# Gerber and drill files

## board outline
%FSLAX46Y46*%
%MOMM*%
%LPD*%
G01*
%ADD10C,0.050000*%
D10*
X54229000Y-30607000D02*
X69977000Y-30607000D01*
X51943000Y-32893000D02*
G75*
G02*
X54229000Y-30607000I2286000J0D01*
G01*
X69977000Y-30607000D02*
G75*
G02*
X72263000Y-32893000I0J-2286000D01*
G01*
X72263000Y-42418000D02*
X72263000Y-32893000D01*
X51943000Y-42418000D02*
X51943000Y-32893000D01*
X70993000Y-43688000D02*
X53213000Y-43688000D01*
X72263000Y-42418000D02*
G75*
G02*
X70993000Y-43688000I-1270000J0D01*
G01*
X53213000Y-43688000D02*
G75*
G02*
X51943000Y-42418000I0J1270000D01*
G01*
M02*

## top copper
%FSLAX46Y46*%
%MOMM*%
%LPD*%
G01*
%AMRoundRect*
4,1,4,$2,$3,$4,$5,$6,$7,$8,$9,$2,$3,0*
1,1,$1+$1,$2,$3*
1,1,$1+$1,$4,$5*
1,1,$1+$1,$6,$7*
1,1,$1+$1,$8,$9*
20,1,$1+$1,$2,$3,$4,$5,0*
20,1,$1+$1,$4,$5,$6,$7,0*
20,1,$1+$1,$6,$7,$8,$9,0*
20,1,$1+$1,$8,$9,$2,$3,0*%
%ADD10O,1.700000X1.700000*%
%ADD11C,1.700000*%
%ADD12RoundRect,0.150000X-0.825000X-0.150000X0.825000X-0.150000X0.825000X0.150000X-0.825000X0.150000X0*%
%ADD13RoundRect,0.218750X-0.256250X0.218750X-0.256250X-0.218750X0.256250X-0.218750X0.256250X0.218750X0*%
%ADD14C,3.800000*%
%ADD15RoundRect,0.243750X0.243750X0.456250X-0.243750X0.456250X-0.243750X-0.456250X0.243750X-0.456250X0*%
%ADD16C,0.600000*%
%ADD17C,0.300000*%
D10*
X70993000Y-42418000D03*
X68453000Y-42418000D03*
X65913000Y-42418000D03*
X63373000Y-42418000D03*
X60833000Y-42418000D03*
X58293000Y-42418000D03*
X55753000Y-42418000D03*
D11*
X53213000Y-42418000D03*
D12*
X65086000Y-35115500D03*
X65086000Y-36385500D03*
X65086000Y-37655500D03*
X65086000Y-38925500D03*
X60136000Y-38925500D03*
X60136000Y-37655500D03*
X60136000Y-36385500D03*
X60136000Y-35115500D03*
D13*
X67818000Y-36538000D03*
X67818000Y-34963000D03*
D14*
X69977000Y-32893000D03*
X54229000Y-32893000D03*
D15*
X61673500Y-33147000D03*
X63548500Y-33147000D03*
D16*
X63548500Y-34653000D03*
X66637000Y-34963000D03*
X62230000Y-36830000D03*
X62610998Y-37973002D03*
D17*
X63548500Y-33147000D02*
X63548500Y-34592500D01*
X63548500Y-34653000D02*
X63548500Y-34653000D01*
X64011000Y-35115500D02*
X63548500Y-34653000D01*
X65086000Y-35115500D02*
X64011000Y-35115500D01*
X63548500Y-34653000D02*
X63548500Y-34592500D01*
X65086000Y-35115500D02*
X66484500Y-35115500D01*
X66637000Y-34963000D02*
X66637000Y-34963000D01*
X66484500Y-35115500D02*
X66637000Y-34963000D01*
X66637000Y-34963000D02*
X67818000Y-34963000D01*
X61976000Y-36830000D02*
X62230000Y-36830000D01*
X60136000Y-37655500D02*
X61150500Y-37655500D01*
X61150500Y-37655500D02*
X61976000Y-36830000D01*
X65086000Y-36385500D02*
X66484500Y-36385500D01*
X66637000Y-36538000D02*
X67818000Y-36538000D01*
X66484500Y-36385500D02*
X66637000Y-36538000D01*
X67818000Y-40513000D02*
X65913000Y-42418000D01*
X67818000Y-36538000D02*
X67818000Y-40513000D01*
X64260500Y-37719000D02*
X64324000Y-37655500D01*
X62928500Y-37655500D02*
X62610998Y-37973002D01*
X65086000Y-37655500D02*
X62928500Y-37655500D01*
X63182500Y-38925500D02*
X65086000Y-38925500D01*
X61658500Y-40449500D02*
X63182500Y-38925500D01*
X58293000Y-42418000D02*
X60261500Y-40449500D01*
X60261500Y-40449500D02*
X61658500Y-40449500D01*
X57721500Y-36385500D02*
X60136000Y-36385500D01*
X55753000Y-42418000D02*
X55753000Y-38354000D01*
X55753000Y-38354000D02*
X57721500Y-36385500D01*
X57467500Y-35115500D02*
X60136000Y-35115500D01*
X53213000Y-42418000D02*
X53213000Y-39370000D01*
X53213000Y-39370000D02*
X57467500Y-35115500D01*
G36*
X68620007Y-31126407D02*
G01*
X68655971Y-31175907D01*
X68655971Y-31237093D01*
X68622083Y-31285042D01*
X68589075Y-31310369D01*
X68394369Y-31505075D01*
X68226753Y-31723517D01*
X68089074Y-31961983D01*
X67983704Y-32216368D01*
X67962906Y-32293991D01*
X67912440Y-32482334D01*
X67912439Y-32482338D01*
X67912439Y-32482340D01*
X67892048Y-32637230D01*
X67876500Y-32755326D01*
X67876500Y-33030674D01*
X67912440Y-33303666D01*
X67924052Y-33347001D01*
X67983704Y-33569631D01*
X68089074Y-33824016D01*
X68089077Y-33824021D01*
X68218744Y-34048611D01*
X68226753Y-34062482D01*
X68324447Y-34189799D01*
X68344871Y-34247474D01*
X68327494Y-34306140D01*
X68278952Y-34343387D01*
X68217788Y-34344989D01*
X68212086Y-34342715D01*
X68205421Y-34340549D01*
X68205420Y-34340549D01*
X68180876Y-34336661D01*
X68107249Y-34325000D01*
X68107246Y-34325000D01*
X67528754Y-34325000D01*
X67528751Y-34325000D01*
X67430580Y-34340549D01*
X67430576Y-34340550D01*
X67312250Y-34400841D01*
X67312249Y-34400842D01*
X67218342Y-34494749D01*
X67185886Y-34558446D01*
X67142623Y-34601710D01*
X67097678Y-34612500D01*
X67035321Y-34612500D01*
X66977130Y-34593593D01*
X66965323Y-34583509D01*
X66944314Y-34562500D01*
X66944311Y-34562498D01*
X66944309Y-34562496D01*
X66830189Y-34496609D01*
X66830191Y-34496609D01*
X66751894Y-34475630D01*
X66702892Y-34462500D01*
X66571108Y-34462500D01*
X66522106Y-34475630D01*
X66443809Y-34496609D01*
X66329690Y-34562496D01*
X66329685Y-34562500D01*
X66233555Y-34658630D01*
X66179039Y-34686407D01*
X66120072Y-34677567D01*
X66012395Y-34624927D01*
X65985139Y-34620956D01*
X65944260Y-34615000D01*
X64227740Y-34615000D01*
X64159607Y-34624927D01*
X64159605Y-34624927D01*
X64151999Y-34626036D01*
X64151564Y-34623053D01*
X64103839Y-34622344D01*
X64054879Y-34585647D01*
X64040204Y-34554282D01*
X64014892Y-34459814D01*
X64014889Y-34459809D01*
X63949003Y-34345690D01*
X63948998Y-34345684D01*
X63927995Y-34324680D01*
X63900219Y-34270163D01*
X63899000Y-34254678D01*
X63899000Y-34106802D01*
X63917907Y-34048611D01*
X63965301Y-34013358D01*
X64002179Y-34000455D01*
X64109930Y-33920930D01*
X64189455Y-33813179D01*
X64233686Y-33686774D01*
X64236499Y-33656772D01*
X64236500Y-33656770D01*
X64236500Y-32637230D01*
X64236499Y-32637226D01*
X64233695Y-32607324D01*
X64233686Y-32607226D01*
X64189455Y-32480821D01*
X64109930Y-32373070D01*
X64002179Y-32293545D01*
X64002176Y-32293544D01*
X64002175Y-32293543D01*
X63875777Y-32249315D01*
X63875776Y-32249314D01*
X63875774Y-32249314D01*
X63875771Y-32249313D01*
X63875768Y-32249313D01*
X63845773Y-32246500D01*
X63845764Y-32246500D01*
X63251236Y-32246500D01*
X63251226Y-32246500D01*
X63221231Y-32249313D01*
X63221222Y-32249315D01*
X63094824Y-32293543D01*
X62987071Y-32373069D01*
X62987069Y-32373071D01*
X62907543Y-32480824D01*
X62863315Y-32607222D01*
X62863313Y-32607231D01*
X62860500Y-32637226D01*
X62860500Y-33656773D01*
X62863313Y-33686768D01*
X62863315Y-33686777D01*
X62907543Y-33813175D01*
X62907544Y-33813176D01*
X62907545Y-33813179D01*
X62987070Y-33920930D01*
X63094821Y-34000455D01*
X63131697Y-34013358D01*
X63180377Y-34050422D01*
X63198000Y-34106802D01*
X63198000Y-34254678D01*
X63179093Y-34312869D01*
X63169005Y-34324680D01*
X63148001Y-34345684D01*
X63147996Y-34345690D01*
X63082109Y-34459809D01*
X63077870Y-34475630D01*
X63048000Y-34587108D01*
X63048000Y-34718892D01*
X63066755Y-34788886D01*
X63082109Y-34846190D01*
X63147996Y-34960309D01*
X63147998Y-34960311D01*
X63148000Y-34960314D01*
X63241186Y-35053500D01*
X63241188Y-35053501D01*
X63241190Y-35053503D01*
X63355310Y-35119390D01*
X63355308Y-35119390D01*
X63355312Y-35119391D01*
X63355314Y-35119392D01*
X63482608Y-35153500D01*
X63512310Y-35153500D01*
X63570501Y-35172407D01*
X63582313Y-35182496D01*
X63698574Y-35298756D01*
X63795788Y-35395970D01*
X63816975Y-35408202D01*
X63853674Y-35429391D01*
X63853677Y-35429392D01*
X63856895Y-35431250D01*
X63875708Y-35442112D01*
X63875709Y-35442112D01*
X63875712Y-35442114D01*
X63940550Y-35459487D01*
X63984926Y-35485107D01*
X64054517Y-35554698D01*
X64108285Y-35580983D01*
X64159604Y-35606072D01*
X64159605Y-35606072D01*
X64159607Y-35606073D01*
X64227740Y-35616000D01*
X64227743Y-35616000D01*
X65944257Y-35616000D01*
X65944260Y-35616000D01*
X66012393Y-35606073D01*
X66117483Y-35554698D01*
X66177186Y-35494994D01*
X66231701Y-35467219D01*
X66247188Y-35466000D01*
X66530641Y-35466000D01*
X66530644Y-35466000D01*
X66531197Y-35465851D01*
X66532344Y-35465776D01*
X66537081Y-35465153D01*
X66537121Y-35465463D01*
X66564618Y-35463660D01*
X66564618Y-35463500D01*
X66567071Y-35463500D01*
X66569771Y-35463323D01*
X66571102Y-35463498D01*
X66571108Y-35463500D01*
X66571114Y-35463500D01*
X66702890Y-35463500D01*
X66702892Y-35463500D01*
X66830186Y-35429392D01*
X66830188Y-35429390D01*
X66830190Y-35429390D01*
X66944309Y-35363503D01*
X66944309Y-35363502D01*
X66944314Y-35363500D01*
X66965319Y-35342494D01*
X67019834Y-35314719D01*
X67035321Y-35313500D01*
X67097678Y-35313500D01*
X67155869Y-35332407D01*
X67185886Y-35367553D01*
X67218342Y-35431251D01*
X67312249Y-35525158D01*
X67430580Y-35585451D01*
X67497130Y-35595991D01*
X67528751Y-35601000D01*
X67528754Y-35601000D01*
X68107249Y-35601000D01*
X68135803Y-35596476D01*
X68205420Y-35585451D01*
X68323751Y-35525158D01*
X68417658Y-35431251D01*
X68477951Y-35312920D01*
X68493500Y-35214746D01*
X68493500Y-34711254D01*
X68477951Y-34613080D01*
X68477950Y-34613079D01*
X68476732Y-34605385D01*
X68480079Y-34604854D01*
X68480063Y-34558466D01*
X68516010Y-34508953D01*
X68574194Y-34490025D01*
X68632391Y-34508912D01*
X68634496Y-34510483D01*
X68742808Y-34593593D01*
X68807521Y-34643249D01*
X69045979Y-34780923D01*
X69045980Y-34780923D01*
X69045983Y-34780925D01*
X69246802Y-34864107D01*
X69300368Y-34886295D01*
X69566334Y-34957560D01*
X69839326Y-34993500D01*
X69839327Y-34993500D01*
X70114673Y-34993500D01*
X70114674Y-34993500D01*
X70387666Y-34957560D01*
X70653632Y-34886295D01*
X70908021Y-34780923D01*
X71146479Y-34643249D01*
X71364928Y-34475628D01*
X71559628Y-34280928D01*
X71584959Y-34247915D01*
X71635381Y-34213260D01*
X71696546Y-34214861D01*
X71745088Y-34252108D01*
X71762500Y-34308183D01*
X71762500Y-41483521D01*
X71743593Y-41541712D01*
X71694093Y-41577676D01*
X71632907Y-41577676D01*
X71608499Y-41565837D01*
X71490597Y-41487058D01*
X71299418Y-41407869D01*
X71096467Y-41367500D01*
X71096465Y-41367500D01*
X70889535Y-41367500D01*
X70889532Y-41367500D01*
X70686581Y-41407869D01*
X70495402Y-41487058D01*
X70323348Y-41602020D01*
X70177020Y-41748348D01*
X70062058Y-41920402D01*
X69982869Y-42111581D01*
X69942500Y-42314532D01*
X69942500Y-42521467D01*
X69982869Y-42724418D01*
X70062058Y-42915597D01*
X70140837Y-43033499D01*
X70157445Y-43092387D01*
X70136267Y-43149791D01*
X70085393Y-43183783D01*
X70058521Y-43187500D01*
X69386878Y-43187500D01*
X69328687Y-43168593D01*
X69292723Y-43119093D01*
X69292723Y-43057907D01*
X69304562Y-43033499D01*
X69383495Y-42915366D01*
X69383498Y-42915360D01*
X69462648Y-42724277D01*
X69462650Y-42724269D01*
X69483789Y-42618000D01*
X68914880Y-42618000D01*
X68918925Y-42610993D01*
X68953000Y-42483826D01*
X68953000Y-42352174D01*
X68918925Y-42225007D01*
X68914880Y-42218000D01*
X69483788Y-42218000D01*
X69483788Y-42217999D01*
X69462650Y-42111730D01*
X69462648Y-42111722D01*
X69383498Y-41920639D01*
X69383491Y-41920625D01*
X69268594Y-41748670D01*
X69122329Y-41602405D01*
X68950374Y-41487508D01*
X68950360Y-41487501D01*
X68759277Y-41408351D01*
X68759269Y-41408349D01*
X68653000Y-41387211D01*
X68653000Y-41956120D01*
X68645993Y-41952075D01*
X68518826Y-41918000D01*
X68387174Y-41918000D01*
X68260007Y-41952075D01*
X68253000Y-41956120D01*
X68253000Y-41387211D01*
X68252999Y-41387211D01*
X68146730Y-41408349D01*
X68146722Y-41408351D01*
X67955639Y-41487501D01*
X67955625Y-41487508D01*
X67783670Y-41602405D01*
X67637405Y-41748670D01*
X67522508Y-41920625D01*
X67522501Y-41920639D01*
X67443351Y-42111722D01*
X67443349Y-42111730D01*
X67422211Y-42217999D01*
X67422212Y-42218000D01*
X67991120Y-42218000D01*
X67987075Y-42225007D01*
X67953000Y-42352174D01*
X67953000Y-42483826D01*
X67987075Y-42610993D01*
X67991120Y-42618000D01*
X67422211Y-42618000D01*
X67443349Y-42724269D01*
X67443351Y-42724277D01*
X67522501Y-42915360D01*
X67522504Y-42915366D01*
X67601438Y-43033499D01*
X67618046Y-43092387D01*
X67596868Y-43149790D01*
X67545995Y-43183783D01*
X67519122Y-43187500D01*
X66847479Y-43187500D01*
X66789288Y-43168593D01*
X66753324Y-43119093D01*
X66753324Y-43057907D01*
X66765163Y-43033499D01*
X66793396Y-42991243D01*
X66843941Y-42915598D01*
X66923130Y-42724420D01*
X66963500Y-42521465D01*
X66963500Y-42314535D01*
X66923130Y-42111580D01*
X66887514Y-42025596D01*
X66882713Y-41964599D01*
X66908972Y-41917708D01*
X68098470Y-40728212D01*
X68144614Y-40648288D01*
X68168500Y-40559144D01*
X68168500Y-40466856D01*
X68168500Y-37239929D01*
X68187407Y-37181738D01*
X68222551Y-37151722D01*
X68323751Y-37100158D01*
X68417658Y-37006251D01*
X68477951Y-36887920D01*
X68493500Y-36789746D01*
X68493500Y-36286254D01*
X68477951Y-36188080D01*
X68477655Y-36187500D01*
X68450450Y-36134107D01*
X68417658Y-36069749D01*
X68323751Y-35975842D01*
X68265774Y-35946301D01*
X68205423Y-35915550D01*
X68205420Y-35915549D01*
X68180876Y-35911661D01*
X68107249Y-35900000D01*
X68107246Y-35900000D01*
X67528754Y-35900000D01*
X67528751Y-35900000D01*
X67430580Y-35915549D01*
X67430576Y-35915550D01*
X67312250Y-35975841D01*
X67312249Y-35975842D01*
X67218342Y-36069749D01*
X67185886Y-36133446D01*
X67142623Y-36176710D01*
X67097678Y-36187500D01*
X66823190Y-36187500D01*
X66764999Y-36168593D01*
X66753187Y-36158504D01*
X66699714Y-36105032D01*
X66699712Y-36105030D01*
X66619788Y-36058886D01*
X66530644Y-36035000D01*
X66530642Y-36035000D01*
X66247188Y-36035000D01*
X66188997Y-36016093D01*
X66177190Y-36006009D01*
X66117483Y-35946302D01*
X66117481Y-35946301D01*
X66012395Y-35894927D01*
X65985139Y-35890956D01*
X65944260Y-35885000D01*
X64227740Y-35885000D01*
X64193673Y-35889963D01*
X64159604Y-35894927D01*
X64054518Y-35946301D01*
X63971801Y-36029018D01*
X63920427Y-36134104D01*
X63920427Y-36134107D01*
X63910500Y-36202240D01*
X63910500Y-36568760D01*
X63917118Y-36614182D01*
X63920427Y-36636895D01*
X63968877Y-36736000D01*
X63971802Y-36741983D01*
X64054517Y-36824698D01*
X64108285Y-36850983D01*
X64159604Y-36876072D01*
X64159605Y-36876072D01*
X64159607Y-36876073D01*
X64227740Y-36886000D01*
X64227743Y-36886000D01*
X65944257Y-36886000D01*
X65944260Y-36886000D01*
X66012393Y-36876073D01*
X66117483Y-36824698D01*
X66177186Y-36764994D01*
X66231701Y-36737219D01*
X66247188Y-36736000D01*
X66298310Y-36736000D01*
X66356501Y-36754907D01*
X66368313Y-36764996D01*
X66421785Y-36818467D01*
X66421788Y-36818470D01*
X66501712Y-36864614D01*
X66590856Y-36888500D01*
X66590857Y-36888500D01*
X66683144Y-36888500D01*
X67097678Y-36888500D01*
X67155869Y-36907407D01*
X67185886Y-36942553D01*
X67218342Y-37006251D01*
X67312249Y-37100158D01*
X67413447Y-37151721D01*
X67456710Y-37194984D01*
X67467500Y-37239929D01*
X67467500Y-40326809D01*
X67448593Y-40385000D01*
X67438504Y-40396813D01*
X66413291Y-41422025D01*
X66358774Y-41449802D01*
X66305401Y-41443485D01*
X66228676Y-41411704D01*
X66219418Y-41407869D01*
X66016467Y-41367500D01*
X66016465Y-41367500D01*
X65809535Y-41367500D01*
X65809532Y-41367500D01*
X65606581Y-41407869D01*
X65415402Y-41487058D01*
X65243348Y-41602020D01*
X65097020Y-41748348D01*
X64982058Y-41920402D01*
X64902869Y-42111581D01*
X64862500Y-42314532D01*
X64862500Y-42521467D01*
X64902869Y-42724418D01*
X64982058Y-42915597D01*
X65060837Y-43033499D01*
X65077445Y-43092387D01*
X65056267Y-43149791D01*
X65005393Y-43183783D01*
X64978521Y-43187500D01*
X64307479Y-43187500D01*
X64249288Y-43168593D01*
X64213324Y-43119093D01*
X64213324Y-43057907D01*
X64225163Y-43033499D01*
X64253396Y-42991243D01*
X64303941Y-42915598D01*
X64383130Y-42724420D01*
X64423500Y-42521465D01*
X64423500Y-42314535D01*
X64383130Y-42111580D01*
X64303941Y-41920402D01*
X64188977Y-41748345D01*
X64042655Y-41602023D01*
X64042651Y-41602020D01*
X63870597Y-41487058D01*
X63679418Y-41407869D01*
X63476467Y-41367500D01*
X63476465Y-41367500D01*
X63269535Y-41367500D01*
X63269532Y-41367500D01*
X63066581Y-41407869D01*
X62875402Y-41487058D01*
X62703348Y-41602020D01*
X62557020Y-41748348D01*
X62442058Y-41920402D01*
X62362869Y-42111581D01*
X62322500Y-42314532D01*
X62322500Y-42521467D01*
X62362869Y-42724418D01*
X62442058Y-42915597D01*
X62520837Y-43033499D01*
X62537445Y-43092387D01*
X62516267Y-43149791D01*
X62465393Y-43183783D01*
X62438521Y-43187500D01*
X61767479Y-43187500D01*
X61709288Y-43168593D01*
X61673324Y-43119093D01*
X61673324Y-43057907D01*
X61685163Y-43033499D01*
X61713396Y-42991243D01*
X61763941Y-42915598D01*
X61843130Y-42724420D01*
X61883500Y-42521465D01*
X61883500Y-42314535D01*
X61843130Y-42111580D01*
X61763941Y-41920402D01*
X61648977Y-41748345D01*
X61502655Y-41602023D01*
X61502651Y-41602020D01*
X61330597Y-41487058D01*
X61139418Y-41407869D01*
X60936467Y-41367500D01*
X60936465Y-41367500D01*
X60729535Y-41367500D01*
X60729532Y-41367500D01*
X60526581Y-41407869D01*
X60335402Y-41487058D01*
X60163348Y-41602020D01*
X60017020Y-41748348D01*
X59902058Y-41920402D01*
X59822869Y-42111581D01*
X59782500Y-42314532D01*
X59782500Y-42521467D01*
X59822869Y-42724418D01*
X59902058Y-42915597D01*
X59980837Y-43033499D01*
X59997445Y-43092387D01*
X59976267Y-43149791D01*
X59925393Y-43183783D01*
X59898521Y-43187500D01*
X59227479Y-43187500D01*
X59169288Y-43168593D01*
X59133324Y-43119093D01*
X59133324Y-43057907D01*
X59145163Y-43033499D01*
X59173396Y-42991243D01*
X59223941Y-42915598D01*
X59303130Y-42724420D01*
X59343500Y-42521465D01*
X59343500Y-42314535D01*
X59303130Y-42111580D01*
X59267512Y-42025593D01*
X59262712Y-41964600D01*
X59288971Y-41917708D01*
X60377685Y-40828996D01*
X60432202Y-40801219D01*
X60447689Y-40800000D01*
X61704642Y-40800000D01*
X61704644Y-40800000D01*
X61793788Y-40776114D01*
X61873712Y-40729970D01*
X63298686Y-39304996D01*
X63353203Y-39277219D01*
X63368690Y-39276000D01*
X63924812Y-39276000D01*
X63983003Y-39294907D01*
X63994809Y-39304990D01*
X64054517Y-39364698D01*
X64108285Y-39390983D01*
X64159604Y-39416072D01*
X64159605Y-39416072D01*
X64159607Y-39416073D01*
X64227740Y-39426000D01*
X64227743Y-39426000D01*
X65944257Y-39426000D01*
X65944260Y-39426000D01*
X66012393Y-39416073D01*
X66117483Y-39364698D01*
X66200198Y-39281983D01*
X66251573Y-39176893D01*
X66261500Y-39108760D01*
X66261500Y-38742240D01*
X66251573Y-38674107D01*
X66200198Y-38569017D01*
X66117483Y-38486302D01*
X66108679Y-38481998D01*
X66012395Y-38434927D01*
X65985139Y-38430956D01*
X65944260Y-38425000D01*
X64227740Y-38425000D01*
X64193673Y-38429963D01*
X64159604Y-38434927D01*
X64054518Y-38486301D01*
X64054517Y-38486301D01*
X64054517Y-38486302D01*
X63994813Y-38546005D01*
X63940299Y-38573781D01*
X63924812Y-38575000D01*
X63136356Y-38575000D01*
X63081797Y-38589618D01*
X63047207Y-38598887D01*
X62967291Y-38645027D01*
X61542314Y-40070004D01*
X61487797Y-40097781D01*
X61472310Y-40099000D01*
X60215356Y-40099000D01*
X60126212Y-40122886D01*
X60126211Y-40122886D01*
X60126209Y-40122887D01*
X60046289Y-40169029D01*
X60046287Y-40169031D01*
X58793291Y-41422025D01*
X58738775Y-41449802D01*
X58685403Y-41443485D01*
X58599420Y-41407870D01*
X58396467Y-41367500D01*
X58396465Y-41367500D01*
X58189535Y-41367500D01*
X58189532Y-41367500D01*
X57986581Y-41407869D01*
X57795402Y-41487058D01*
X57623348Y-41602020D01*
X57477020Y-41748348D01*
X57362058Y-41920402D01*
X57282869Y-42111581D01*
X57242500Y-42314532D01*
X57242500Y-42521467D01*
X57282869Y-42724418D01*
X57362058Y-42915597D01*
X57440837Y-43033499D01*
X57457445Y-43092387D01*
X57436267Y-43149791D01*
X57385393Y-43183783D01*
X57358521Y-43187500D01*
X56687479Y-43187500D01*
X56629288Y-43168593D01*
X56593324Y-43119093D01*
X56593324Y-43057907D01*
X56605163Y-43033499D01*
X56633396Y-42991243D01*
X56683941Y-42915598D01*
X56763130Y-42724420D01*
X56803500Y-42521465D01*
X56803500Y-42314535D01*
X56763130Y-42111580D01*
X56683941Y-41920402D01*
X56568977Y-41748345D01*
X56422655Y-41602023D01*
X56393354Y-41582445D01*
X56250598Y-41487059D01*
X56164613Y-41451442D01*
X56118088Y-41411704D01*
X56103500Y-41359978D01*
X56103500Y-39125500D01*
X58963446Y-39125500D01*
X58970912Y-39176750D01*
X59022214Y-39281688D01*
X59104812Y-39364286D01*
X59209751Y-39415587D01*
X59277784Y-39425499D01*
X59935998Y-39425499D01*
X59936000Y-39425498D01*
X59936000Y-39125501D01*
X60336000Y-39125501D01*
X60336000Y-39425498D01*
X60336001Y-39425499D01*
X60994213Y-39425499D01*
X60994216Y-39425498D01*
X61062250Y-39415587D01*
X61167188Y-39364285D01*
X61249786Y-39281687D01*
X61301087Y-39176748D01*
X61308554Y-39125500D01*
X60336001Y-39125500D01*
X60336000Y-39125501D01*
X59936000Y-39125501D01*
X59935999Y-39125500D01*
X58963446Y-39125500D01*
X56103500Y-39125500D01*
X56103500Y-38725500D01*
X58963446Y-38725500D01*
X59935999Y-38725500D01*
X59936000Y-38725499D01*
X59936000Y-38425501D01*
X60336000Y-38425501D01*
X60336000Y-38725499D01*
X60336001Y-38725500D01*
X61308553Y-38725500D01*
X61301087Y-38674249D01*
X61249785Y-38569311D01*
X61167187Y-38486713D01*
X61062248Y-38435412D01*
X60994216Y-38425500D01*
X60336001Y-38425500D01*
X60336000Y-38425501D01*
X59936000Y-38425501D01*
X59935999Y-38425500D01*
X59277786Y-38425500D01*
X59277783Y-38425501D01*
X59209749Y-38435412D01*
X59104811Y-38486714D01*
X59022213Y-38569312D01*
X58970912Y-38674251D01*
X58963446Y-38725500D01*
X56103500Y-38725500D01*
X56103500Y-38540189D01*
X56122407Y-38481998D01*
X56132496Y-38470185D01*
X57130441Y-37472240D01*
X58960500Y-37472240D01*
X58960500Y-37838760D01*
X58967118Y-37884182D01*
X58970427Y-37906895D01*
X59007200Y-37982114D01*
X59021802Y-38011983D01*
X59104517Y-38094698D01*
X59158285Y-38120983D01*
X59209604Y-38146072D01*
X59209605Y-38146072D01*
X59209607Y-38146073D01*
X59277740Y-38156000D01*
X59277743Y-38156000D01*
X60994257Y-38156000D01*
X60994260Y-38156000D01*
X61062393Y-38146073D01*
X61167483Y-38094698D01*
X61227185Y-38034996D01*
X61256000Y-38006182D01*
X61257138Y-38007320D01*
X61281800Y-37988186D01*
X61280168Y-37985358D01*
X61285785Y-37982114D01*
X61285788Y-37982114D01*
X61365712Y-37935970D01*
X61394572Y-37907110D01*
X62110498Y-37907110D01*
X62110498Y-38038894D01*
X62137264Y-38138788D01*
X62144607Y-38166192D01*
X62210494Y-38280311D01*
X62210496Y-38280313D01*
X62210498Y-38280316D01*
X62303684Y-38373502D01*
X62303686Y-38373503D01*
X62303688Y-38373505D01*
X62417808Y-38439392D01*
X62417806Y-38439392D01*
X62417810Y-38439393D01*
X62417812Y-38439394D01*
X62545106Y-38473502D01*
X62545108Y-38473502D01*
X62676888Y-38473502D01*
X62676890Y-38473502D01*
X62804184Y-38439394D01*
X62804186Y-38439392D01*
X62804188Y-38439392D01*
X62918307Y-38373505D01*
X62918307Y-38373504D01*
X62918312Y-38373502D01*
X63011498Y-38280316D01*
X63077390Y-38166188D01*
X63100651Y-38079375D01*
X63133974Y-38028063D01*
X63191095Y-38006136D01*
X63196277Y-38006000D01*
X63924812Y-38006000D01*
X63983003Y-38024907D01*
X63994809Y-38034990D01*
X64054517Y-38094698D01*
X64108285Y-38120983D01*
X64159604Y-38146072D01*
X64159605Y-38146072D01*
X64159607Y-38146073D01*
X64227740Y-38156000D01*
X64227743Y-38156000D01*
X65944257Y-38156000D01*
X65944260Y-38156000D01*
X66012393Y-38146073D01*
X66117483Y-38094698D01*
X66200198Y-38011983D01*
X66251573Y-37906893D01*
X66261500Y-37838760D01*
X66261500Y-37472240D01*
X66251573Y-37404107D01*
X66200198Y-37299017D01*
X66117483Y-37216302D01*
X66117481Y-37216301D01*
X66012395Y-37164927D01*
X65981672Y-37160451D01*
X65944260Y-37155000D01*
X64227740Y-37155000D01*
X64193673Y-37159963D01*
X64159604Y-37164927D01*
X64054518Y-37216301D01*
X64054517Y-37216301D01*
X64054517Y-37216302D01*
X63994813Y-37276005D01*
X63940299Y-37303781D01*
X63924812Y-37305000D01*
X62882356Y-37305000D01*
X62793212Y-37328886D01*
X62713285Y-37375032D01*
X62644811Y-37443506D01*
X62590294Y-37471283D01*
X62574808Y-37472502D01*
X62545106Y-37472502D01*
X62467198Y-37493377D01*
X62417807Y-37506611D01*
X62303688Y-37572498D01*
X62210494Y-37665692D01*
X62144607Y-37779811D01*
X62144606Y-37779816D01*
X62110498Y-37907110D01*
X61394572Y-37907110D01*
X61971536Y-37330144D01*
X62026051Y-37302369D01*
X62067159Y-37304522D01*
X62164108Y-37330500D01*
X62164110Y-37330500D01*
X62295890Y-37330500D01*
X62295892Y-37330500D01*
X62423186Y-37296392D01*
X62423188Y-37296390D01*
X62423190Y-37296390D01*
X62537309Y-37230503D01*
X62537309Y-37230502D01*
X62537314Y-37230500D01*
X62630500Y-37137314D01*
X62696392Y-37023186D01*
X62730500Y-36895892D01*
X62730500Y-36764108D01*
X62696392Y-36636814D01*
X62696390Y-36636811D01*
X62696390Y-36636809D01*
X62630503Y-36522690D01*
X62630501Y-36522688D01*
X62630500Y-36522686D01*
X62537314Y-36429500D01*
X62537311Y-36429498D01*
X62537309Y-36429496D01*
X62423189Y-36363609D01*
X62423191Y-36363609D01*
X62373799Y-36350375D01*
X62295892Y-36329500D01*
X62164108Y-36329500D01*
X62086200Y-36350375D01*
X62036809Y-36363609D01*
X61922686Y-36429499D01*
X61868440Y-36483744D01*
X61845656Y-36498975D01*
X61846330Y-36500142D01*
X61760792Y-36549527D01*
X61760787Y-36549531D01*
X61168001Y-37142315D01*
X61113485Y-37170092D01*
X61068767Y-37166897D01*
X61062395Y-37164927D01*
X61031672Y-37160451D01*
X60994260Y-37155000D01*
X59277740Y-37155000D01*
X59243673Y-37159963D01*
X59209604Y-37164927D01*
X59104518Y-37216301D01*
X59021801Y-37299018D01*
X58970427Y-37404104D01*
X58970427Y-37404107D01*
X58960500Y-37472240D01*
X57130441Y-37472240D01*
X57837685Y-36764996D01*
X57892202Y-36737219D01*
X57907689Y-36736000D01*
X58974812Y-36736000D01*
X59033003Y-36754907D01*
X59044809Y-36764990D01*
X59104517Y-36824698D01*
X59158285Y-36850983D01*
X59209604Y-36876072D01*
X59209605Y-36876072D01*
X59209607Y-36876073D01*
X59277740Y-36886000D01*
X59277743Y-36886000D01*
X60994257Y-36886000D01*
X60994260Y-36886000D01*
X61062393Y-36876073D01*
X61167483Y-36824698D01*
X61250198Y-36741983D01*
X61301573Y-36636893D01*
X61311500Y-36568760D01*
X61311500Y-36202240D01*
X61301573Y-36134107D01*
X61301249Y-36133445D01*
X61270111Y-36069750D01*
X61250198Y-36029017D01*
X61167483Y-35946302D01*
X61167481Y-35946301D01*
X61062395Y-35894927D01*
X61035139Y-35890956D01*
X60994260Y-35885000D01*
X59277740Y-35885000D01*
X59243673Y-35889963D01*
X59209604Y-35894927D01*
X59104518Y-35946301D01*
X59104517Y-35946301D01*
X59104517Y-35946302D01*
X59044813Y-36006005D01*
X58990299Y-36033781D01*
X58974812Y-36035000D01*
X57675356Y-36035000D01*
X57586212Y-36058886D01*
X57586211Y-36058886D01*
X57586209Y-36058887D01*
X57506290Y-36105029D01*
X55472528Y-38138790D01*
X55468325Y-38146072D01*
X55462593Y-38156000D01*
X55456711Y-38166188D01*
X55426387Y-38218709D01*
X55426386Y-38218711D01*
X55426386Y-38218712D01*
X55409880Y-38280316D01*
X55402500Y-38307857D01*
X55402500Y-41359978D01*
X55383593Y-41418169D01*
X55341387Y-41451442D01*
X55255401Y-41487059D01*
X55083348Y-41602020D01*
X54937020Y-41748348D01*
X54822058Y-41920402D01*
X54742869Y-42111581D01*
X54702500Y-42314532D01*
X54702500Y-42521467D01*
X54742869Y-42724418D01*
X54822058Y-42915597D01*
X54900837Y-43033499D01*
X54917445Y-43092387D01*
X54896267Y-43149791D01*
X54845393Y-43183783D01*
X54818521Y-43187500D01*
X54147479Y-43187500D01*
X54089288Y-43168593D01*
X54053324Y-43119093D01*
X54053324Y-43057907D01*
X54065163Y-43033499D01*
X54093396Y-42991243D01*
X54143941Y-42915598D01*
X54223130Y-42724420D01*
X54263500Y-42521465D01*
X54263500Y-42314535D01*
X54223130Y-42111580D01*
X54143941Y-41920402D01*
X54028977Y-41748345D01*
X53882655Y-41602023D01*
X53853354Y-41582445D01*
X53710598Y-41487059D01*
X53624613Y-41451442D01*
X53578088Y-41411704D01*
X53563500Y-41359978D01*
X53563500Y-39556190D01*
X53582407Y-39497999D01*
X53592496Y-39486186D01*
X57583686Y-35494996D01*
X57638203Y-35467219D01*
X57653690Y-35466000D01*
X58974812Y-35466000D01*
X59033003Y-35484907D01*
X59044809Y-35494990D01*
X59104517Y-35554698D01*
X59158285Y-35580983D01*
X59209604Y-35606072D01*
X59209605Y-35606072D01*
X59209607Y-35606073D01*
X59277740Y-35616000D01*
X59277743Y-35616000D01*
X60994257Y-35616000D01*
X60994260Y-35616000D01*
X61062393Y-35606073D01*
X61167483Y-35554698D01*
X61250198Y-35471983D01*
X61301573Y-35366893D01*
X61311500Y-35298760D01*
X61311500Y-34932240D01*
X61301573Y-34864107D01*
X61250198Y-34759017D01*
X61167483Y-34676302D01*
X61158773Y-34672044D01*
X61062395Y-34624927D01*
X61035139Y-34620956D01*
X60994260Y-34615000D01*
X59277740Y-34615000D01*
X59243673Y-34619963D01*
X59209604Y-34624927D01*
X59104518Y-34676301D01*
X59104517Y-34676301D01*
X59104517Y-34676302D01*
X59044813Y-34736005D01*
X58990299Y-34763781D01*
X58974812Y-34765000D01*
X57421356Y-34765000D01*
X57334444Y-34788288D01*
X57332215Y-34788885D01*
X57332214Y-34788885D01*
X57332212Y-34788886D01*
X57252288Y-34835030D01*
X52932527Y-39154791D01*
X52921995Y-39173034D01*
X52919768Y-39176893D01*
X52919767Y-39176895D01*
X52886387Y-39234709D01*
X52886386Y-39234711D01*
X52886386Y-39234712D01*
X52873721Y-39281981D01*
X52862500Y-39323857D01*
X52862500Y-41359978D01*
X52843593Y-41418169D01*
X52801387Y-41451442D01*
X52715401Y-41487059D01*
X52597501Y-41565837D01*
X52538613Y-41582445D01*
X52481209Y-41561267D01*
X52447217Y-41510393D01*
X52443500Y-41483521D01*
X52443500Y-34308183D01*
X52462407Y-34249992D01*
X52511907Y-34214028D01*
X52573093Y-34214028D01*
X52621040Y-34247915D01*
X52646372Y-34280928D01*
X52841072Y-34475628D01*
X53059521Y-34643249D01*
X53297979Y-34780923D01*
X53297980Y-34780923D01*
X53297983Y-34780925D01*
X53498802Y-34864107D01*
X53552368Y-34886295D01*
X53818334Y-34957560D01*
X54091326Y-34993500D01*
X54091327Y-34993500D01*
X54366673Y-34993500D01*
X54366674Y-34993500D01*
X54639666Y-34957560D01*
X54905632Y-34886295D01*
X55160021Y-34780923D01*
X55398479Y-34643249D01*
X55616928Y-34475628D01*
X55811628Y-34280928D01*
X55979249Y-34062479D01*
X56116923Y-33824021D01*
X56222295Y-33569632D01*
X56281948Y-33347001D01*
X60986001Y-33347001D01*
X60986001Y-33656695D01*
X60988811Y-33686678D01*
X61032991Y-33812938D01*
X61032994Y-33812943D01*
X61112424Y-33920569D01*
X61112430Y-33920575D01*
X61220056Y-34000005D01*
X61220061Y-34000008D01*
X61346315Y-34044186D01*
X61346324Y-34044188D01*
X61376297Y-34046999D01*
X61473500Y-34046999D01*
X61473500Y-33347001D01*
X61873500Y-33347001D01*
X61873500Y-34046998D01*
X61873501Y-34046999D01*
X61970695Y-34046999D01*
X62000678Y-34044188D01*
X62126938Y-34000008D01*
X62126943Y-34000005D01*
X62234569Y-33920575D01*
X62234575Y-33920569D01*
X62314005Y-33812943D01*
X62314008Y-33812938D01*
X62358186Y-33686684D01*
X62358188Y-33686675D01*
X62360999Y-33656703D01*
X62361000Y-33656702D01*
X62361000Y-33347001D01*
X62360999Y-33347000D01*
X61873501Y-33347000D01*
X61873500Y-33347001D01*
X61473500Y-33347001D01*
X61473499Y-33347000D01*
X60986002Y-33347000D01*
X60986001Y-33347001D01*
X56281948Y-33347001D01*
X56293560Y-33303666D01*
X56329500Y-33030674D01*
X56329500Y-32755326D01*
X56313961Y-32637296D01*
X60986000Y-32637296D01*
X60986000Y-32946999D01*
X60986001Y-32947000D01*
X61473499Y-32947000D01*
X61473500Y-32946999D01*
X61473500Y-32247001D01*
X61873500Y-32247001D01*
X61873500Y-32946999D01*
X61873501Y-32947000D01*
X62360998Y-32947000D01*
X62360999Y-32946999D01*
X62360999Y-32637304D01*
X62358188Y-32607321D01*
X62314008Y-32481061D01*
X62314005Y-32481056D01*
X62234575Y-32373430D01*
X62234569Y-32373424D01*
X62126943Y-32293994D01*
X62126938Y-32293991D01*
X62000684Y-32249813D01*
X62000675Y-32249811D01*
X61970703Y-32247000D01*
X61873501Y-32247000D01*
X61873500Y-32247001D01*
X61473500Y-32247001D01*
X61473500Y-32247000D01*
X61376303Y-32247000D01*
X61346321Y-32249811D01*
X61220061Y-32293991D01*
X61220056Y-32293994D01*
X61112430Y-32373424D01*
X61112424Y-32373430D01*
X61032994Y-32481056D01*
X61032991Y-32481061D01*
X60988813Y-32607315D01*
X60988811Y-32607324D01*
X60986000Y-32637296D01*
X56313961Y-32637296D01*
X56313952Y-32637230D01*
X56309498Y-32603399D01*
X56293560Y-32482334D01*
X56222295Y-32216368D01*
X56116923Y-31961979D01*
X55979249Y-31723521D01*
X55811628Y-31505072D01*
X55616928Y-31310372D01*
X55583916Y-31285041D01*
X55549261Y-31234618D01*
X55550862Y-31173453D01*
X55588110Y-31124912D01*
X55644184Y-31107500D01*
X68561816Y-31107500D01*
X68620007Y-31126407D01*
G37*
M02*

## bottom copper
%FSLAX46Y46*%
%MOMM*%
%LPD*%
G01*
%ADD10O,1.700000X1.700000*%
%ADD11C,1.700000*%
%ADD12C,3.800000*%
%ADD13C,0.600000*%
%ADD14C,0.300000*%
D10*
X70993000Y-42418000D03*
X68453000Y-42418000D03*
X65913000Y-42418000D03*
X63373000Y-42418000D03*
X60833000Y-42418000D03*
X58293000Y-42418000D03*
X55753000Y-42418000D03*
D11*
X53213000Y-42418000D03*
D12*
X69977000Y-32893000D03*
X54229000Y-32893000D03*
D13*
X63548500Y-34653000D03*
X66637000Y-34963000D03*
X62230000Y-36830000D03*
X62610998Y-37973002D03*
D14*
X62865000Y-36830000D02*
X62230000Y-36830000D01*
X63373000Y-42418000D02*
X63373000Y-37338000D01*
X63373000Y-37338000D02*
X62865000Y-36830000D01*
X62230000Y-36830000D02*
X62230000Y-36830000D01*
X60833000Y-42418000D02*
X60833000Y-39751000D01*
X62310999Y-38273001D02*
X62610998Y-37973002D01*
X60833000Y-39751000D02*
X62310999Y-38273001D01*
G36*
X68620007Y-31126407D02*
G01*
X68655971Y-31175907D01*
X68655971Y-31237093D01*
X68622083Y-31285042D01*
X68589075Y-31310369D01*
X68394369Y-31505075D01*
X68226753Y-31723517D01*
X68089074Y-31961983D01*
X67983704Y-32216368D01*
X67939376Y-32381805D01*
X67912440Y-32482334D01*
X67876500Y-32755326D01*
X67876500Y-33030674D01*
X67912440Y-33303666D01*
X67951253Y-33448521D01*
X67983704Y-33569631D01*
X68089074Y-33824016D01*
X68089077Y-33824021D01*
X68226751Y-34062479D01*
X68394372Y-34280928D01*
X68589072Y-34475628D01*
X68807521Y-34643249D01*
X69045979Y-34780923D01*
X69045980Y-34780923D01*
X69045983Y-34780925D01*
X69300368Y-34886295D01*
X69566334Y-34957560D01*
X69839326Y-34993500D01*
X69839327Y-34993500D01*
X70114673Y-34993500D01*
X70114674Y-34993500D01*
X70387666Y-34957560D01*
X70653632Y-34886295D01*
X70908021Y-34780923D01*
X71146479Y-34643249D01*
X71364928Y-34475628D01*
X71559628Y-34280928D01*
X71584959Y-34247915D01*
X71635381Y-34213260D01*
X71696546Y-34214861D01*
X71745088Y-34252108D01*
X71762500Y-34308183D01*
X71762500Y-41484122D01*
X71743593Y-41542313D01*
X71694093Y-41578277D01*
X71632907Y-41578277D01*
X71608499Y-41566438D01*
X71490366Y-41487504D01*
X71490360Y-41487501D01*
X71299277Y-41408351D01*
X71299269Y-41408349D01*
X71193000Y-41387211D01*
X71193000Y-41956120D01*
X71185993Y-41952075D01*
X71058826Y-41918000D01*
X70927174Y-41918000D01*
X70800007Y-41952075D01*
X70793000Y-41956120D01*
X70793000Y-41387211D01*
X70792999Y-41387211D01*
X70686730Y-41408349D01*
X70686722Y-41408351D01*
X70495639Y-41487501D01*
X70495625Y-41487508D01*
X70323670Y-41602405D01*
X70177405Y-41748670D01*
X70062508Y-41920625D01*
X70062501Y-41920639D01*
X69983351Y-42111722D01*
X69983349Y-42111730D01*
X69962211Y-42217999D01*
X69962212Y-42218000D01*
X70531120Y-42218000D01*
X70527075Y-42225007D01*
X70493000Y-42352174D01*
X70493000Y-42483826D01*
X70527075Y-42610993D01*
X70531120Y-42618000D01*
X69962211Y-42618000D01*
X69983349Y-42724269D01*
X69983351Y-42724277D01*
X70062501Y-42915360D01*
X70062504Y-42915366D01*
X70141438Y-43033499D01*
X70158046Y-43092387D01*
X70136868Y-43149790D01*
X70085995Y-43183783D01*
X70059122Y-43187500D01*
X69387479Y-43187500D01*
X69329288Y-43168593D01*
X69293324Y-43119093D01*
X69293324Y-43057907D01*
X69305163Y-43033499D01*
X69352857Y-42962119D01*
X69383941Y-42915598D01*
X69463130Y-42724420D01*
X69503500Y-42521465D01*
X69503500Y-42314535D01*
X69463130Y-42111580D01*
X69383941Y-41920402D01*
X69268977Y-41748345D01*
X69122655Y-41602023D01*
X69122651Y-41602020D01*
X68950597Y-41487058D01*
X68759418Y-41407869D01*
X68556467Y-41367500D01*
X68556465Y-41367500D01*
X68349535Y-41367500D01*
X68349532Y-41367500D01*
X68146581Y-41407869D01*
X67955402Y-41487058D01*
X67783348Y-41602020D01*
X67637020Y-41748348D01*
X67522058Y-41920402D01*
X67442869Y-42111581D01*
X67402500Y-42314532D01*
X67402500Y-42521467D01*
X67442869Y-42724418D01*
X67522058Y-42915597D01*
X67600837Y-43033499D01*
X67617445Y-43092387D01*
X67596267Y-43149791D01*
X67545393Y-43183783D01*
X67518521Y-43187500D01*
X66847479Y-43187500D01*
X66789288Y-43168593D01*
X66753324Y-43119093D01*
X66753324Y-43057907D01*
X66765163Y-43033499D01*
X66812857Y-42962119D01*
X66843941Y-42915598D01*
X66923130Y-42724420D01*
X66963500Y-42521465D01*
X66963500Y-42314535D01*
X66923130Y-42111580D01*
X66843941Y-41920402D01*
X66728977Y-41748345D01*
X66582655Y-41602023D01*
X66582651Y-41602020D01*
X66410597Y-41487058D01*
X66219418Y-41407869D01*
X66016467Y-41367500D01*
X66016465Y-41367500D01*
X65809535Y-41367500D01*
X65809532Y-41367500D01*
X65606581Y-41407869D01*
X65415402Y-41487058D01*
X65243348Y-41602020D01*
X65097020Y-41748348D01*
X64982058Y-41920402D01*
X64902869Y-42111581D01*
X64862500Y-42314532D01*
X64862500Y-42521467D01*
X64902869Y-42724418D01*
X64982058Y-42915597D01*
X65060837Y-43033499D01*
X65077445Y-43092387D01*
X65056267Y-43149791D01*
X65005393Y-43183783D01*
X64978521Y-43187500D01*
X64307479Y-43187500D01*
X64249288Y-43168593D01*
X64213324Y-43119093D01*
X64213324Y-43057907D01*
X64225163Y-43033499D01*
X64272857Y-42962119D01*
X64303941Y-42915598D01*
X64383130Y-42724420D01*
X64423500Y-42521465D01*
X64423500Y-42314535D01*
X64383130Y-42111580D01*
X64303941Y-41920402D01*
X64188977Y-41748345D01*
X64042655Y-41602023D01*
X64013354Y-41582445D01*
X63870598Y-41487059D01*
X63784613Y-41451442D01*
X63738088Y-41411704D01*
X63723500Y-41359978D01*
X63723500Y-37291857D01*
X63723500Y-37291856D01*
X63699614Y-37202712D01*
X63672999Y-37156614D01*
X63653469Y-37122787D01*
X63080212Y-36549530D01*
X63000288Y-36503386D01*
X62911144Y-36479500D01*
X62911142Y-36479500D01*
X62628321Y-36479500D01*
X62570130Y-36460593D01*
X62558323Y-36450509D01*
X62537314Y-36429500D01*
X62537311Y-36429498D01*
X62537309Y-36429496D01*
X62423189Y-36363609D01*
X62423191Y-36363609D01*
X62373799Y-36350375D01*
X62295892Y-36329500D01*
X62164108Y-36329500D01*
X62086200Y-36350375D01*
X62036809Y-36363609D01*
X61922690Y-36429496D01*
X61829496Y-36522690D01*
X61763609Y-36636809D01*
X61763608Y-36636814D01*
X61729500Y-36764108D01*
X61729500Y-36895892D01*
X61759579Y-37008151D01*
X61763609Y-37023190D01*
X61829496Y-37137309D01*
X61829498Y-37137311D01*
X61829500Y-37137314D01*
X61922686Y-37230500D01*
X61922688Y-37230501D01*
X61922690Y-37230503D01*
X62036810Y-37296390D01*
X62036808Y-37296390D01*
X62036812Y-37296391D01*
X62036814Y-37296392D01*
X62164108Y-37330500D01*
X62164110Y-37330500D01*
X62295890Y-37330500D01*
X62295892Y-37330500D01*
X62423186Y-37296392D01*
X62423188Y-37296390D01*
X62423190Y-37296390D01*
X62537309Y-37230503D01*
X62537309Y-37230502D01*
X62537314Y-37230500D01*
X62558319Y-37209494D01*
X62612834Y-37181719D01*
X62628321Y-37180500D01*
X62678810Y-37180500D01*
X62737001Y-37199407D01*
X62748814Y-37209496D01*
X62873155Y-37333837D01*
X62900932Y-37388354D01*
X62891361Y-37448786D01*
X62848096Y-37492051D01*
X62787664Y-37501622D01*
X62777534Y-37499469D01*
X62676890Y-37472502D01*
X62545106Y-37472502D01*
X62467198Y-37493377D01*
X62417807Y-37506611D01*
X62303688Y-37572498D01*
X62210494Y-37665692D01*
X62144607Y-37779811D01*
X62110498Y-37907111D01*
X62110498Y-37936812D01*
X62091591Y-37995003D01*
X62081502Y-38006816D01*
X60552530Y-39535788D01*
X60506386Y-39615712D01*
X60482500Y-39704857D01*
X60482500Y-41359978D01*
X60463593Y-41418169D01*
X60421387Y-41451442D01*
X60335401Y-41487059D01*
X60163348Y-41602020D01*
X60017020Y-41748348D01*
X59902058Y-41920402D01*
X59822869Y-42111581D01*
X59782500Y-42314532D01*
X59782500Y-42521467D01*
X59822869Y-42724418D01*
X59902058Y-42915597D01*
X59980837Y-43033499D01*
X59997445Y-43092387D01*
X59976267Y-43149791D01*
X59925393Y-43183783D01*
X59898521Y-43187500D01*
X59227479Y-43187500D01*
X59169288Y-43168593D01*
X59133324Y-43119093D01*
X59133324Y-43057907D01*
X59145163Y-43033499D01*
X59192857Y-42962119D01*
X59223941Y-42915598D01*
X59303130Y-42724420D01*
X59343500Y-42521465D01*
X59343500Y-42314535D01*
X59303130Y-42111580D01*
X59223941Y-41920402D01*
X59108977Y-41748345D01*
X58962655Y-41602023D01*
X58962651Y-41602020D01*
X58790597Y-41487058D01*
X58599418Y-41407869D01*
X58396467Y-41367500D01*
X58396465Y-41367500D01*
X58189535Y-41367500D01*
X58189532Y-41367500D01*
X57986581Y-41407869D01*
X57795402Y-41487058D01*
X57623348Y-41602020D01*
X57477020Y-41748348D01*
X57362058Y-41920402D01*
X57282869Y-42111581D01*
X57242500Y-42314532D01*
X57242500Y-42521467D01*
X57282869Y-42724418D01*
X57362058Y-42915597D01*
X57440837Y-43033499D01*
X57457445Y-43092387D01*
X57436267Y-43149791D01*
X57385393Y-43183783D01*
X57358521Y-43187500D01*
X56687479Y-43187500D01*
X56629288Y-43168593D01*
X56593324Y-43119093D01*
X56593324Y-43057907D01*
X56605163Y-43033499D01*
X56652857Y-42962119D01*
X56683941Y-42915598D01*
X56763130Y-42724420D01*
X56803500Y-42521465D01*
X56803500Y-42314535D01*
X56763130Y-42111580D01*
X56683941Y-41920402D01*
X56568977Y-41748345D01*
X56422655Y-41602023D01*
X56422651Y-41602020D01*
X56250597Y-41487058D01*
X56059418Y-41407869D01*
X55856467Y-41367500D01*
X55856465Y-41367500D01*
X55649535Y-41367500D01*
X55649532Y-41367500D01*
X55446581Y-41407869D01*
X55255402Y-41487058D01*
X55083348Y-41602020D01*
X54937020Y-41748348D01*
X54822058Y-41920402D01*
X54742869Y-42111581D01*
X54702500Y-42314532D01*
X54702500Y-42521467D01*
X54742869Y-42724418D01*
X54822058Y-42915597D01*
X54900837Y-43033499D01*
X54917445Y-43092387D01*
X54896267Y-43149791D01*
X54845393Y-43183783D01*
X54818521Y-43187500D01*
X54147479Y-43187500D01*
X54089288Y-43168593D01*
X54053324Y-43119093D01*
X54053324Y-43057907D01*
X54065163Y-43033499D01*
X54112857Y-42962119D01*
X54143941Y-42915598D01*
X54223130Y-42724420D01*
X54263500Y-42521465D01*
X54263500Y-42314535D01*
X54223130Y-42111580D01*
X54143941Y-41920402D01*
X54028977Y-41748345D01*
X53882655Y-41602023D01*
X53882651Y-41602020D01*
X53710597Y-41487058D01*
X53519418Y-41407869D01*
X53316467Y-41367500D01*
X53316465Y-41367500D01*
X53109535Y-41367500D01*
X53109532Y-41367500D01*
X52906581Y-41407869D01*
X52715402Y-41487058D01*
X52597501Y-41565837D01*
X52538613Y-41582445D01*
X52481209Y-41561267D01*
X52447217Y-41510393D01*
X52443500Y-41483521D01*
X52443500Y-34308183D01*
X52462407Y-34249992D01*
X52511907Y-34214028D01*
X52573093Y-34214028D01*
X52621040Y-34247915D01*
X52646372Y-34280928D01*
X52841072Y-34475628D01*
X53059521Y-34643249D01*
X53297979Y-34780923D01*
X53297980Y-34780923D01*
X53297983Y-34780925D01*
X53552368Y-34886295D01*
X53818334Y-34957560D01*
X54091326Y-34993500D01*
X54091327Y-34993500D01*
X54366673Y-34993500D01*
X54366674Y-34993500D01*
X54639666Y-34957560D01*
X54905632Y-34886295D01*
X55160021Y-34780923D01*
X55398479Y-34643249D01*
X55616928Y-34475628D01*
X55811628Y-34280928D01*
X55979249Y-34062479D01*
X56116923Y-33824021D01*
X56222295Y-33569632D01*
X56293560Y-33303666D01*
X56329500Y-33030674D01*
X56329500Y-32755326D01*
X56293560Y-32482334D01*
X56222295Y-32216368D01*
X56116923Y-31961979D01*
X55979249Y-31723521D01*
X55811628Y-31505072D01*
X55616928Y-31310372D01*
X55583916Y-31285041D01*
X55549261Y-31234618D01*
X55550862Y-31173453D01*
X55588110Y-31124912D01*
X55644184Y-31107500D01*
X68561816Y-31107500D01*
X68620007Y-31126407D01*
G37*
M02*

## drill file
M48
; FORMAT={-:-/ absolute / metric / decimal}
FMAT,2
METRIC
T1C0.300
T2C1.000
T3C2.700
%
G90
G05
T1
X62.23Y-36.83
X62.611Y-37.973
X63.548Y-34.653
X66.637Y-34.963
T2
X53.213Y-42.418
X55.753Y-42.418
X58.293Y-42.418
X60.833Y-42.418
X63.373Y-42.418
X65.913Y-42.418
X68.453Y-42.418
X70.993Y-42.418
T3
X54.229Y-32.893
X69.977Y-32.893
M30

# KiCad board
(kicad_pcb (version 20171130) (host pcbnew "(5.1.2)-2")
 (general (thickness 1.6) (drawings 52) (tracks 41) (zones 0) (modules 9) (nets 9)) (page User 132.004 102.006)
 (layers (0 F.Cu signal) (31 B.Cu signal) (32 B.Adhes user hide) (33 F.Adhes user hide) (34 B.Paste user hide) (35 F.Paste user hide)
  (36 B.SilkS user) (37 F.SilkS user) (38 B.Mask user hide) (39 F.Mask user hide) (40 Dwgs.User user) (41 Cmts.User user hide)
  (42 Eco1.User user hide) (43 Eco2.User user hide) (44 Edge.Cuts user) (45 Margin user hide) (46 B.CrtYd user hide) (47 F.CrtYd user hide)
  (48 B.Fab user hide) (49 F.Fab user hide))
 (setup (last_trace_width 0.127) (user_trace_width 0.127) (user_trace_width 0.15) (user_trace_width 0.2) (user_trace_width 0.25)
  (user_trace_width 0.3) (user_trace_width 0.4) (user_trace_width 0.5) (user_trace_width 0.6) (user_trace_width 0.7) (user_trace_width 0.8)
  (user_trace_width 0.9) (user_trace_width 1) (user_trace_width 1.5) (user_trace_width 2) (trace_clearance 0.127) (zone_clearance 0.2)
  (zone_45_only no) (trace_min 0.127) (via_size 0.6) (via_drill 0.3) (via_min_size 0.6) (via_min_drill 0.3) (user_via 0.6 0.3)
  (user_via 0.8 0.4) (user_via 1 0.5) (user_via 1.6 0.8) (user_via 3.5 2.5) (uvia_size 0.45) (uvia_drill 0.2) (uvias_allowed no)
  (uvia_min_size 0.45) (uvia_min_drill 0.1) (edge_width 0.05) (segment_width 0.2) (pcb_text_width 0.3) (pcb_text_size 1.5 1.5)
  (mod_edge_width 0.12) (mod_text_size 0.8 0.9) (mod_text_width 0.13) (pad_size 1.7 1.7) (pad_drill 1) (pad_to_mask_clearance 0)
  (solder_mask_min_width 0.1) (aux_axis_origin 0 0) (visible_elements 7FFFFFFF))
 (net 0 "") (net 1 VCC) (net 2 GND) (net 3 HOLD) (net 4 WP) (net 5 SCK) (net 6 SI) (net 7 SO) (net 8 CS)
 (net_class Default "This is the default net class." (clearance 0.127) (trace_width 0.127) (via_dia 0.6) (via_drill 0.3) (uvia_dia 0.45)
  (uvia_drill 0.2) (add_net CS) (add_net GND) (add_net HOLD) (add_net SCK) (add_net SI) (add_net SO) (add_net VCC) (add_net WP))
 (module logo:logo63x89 (layer B.Cu) (at 62.103 37.973)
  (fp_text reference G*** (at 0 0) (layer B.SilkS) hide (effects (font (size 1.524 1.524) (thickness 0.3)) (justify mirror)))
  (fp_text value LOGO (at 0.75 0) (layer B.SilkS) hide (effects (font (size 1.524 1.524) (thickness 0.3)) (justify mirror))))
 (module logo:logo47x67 (layer F.Cu) (at 70.104 37.592)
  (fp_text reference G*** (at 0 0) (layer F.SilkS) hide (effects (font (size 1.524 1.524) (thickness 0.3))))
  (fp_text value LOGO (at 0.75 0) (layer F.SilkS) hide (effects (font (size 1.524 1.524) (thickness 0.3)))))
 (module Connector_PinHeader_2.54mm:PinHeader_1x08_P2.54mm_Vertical (layer B.Cu) (at 53.213 42.418 270)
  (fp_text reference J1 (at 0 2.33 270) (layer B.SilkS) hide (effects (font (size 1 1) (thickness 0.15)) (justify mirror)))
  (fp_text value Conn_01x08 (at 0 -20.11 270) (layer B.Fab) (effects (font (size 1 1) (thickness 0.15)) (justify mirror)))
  (pad 8 thru_hole oval (at 0 -17.78 270) (size 1.7 1.7) (drill 1) (layers *.Cu *.Mask) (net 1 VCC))
  (pad 7 thru_hole oval (at 0 -15.24 270) (size 1.7 1.7) (drill 1) (layers *.Cu *.Mask) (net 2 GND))
  (pad 6 thru_hole oval (at 0 -12.7 270) (size 1.7 1.7) (drill 1) (layers *.Cu *.Mask) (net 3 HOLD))
  (pad 5 thru_hole oval (at 0 -10.16 270) (size 1.7 1.7) (drill 1) (layers *.Cu *.Mask) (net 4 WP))
  (pad 4 thru_hole oval (at 0 -7.62 270) (size 1.7 1.7) (drill 1) (layers *.Cu *.Mask) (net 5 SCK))
  (pad 3 thru_hole oval (at 0 -5.08 270) (size 1.7 1.7) (drill 1) (layers *.Cu *.Mask) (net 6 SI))
  (pad 2 thru_hole oval (at 0 -2.54 270) (size 1.7 1.7) (drill 1) (layers *.Cu *.Mask) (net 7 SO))
  (pad 1 thru_hole circle (at 0 0 270) (size 1.7 1.7) (drill 1) (layers *.Cu *.Mask) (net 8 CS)))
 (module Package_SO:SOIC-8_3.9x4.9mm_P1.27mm (layer F.Cu) (at 62.611 37.0205)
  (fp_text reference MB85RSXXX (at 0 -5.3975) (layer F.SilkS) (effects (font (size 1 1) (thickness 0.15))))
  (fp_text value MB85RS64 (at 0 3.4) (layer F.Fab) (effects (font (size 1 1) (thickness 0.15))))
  (pad 8 smd roundrect (at 2.475 -1.905) (size 1.95 0.6) (layers F.Cu F.Paste F.Mask) (roundrect_rratio 0.25) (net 1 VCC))
  (pad 7 smd roundrect (at 2.475 -0.635) (size 1.95 0.6) (layers F.Cu F.Paste F.Mask) (roundrect_rratio 0.25) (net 3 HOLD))
  (pad 6 smd roundrect (at 2.475 0.635) (size 1.95 0.6) (layers F.Cu F.Paste F.Mask) (roundrect_rratio 0.25) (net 5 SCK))
  (pad 5 smd roundrect (at 2.475 1.905) (size 1.95 0.6) (layers F.Cu F.Paste F.Mask) (roundrect_rratio 0.25) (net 6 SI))
  (pad 4 smd roundrect (at -2.475 1.905) (size 1.95 0.6) (layers F.Cu F.Paste F.Mask) (roundrect_rratio 0.25) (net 2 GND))
  (pad 3 smd roundrect (at -2.475 0.635) (size 1.95 0.6) (layers F.Cu F.Paste F.Mask) (roundrect_rratio 0.25) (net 4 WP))
  (pad 2 smd roundrect (at -2.475 -0.635) (size 1.95 0.6) (layers F.Cu F.Paste F.Mask) (roundrect_rratio 0.25) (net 7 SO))
  (pad 1 smd roundrect (at -2.475 -1.905) (size 1.95 0.6) (layers F.Cu F.Paste F.Mask) (roundrect_rratio 0.25) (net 8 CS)))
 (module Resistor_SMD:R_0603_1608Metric (layer F.Cu) (at 67.818 35.7505 270)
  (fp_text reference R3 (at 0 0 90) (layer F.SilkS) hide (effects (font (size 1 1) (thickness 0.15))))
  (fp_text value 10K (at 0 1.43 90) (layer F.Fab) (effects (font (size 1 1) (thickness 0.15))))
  (pad 2 smd roundrect (at 0.7875 0 270) (size 0.875 0.95) (layers F.Cu F.Paste F.Mask) (roundrect_rratio 0.25) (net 3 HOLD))
  (pad 1 smd roundrect (at -0.7875 0 270) (size 0.875 0.95) (layers F.Cu F.Paste F.Mask) (roundrect_rratio 0.25) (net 1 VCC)))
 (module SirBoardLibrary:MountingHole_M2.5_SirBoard (layer F.Cu) (at 69.977 32.893)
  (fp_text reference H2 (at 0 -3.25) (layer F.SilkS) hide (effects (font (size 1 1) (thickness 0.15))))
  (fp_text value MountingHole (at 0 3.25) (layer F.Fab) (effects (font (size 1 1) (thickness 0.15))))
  (pad 1 thru_hole circle (at 0 0) (size 3.8 3.8) (drill 2.7) (layers *.Cu *.Mask)))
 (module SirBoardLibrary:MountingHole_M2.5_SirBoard (layer F.Cu) (at 54.229 32.893)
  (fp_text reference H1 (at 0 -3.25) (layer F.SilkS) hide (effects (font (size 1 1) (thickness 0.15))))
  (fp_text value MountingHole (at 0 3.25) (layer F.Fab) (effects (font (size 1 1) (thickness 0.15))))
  (pad 1 thru_hole circle (at 0 0) (size 3.8 3.8) (drill 2.7) (layers *.Cu *.Mask)))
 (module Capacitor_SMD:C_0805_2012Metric (layer F.Cu) (at 62.611 33.147 180)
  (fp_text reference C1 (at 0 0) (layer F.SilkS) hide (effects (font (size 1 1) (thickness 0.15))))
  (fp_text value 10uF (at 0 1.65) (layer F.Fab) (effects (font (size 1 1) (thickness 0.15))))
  (pad 2 smd roundrect (at 0.9375 0 180) (size 0.975 1.4) (layers F.Cu F.Paste F.Mask) (roundrect_rratio 0.25) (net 2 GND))
  (pad 1 smd roundrect (at -0.9375 0 180) (size 0.975 1.4) (layers F.Cu F.Paste F.Mask) (roundrect_rratio 0.25) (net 1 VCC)))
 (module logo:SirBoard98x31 (layer B.Cu) (at 62.103 32.766)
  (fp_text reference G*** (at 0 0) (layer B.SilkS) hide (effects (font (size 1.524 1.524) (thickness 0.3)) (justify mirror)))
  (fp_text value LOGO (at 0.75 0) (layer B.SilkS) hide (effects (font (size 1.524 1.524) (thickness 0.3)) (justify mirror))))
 (gr_line (start 54.229 30.607) (end 69.977 30.607) (layer Edge.Cuts) (width 0.05))
 (gr_arc (start 54.229 32.893) (end 54.229 30.607) (angle -90) (layer Edge.Cuts) (width 0.05))
 (gr_arc (start 69.977 32.893) (end 72.263 32.893) (angle -90) (layer Edge.Cuts) (width 0.05))
 (gr_line (start 72.263 42.418) (end 72.263 32.893) (layer Edge.Cuts) (width 0.05))
 (gr_line (start 51.943 42.418) (end 51.943 32.893) (layer Edge.Cuts) (width 0.05))
 (gr_line (start 70.993 43.688) (end 53.213 43.688) (layer Edge.Cuts) (width 0.05))
 (gr_arc (start 70.993 42.418) (end 70.993 43.688) (angle -90) (layer Edge.Cuts) (width 0.05))
 (gr_arc (start 53.213 42.418) (end 51.943 42.418) (angle -90) (layer Edge.Cuts) (width 0.05))
 (segment (start 63.5485 33.147) (end 63.5485 34.5925) (width 0.3) (layer F.Cu) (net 1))
 (segment (start 63.5485 34.653) (end 63.5485 34.653) (width 0.3) (layer F.Cu) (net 1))
 (segment (start 64.011 35.1155) (end 63.5485 34.653) (width 0.3) (layer F.Cu) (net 1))
 (segment (start 65.086 35.1155) (end 64.011 35.1155) (width 0.3) (layer F.Cu) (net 1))
 (segment (start 63.5485 34.653) (end 63.5485 34.5925) (width 0.3) (layer F.Cu) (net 1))
 (via (at 63.5485 34.653) (size 0.6) (drill 0.3) (layers F.Cu B.Cu) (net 1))
 (segment (start 65.086 35.1155) (end 66.4845 35.1155) (width 0.3) (layer F.Cu) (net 1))
 (segment (start 66.637 34.963) (end 66.637 34.963) (width 0.3) (layer F.Cu) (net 1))
 (segment (start 66.4845 35.1155) (end 66.637 34.963) (width 0.3) (layer F.Cu) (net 1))
 (segment (start 66.637 34.963) (end 67.818 34.963) (width 0.3) (layer F.Cu) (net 1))
 (via (at 66.637 34.963) (size 0.6) (drill 0.3) (layers F.Cu B.Cu) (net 1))
 (segment (start 62.865 36.83) (end 62.23 36.83) (width 0.3) (layer B.Cu) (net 4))
 (segment (start 63.373 42.418) (end 63.373 37.338) (width 0.3) (layer B.Cu) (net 4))
 (segment (start 63.373 37.338) (end 62.865 36.83) (width 0.3) (layer B.Cu) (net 4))
 (segment (start 62.23 36.83) (end 62.23 36.83) (width 0.3) (layer B.Cu) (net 4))
 (via (at 62.23 36.83) (size 0.6) (drill 0.3) (layers F.Cu B.Cu) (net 4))
 (segment (start 61.976 36.83) (end 62.23 36.83) (width 0.3) (layer F.Cu) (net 4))
 (segment (start 60.136 37.6555) (end 61.1505 37.6555) (width 0.3) (layer F.Cu) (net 4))
 (segment (start 61.1505 37.6555) (end 61.976 36.83) (width 0.3) (layer F.Cu) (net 4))
 (segment (start 65.086 36.3855) (end 66.4845 36.3855) (width 0.3) (layer F.Cu) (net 3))
 (segment (start 66.637 36.538) (end 67.818 36.538) (width 0.3) (layer F.Cu) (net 3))
 (segment (start 66.4845 36.3855) (end 66.637 36.538) (width 0.3) (layer F.Cu) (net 3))
 (segment (start 67.818 40.513) (end 65.913 42.418) (width 0.3) (layer F.Cu) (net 3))
 (segment (start 67.818 36.538) (end 67.818 40.513) (width 0.3) (layer F.Cu) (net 3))
 (segment (start 64.2605 37.719) (end 64.324 37.6555) (width 0.3) (layer F.Cu) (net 5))
 (via (at 62.610998 37.973002) (size 0.6) (drill 0.3) (layers F.Cu B.Cu) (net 5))
 (segment (start 60.833 42.418) (end 60.833 39.751) (width 0.3) (layer B.Cu) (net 5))
 (segment (start 62.310999 38.273001) (end 62.610998 37.973002) (width 0.3) (layer B.Cu) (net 5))
 (segment (start 60.833 39.751) (end 62.310999 38.273001) (width 0.3) (layer B.Cu) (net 5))
 (segment (start 62.9285 37.6555) (end 62.610998 37.973002) (width 0.3) (layer F.Cu) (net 5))
 (segment (start 65.086 37.6555) (end 62.9285 37.6555) (width 0.3) (layer F.Cu) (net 5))
 (segment (start 63.1825 38.9255) (end 65.086 38.9255) (width 0.3) (layer F.Cu) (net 6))
 (segment (start 61.6585 40.4495) (end 63.1825 38.9255) (width 0.3) (layer F.Cu) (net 6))
 (segment (start 58.293 42.418) (end 60.2615 40.4495) (width 0.3) (layer F.Cu) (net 6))
 (segment (start 60.2615 40.4495) (end 61.6585 40.4495) (width 0.3) (layer F.Cu) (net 6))
 (segment (start 57.7215 36.3855) (end 60.136 36.3855) (width 0.3) (layer F.Cu) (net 7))
 (segment (start 55.753 42.418) (end 55.753 38.354) (width 0.3) (layer F.Cu) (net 7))
 (segment (start 55.753 38.354) (end 57.7215 36.3855) (width 0.3) (layer F.Cu) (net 7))
 (segment (start 57.4675 35.1155) (end 60.136 35.1155) (width 0.3) (layer F.Cu) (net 8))
 (segment (start 53.213 42.418) (end 53.213 39.37) (width 0.3) (layer F.Cu) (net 8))
 (segment (start 53.213 39.37) (end 57.4675 35.1155) (width 0.3) (layer F.Cu) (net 8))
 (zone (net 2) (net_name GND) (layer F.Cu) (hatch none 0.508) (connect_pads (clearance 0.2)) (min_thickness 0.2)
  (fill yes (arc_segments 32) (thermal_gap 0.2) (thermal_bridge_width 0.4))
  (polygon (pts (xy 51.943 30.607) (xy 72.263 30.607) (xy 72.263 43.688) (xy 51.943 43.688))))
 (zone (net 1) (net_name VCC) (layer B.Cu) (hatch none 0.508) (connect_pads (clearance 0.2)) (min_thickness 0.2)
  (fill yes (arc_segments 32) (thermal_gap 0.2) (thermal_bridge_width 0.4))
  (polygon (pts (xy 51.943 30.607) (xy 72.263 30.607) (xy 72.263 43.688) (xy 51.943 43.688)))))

